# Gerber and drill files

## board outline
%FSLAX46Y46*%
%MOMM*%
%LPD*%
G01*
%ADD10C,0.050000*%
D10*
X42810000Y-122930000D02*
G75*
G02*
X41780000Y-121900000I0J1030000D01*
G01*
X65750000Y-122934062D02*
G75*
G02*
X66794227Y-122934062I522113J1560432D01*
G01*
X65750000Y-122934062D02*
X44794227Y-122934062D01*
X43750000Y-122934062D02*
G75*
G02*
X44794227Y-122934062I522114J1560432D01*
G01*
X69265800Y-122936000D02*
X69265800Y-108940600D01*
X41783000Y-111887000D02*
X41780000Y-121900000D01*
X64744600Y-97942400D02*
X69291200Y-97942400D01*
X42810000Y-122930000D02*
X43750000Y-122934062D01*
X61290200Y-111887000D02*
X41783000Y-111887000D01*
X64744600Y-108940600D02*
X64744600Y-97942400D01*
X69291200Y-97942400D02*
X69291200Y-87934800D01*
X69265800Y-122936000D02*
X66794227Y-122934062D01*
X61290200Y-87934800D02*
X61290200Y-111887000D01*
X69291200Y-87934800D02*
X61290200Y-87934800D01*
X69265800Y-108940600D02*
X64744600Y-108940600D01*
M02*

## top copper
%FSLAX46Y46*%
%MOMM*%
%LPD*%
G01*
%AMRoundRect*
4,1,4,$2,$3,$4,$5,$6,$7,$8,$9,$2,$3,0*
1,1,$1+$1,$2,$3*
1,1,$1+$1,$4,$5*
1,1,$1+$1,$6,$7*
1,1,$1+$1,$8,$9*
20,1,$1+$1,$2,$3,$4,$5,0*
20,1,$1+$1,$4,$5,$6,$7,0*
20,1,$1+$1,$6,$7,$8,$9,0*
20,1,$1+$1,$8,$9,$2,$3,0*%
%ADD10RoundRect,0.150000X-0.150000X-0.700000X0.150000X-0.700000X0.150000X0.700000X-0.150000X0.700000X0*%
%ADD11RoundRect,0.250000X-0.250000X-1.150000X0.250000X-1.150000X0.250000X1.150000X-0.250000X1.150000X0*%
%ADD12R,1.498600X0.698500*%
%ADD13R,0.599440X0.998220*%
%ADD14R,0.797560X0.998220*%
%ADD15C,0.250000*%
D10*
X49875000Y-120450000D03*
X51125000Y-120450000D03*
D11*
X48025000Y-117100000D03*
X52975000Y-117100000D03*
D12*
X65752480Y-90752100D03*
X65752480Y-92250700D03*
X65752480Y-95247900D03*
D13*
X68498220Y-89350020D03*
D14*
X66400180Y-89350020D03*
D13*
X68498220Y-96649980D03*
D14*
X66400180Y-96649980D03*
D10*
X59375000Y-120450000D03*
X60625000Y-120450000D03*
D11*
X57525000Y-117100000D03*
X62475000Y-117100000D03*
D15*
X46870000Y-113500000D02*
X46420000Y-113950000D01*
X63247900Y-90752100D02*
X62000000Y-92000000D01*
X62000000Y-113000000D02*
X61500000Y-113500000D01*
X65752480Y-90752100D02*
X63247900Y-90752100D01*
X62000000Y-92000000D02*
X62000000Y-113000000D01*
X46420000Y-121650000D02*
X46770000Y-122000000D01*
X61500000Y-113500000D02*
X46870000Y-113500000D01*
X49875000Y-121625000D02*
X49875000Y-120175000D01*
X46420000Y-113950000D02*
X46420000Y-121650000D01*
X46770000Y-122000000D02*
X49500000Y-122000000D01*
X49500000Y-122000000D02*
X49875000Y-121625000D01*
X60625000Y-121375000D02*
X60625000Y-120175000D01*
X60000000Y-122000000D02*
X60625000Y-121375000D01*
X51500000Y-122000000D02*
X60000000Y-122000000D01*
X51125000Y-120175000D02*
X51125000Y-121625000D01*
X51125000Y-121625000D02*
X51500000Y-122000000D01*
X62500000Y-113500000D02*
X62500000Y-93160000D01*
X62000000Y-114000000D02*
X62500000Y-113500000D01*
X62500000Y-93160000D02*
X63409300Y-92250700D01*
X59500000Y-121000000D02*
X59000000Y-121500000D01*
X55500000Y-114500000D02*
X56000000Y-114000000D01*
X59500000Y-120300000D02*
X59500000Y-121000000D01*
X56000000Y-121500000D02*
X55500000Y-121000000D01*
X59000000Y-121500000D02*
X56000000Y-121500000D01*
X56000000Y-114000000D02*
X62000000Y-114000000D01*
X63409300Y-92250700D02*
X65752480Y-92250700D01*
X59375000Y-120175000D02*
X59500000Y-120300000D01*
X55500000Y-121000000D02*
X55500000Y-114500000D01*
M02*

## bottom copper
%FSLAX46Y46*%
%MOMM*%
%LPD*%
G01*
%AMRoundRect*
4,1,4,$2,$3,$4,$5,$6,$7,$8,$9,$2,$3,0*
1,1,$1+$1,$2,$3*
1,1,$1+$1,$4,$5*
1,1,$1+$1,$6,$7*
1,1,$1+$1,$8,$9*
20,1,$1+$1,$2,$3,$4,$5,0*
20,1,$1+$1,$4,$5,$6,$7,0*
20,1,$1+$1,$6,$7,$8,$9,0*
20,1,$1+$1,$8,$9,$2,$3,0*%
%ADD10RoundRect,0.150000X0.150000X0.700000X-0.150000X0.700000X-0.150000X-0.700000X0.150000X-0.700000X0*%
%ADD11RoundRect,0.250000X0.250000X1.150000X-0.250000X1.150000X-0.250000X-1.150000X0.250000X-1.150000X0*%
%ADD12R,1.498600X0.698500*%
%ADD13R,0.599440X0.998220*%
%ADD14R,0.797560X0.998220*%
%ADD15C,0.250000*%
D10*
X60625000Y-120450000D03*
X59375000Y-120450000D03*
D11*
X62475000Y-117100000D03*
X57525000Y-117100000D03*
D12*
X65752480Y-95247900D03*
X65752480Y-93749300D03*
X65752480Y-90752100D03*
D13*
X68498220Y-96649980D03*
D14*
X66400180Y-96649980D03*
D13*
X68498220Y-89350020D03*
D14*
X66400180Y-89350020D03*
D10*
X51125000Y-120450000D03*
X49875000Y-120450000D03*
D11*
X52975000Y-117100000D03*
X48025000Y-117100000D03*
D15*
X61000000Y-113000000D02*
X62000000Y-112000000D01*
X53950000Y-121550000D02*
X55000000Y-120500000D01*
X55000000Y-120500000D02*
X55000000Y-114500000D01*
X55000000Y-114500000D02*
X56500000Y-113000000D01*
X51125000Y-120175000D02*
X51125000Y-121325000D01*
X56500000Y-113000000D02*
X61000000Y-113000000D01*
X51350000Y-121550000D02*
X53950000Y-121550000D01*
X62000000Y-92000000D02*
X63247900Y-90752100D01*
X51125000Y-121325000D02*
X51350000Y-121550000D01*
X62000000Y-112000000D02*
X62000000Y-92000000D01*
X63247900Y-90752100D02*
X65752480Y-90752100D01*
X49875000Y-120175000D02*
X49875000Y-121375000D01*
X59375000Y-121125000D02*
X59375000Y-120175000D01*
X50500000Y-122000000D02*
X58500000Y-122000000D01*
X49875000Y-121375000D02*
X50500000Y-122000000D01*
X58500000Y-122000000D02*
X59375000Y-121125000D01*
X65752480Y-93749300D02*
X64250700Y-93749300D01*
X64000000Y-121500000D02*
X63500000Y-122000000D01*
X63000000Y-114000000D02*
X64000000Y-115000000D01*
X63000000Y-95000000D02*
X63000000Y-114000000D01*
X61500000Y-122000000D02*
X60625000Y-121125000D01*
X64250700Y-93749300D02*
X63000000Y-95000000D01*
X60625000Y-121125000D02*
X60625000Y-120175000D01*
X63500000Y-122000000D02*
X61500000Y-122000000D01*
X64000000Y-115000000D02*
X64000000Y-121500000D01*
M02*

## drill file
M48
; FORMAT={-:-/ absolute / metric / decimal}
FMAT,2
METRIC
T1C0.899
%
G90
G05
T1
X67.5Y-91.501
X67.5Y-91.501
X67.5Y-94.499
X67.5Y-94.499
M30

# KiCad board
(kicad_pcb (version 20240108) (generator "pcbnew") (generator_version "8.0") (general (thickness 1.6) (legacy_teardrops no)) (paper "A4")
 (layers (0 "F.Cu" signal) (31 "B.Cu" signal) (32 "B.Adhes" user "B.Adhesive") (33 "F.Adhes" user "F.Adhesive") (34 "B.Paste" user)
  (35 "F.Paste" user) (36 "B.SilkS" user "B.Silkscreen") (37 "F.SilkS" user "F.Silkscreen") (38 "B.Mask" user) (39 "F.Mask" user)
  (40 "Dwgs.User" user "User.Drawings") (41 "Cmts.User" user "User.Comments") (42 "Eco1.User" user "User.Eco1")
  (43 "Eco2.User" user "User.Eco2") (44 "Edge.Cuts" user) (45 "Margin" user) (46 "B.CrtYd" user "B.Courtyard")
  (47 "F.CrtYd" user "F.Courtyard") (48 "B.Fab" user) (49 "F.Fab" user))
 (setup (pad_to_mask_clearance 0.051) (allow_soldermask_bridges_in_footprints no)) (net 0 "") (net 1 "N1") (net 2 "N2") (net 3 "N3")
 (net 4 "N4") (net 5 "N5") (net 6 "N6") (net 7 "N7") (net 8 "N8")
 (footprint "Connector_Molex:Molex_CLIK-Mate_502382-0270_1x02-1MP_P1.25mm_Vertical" (layer "F.Cu") (at 50.5 118.5)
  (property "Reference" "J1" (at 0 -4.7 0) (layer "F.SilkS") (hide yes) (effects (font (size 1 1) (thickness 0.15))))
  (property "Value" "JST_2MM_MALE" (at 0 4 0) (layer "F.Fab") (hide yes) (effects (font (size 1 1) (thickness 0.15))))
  (pad "1" smd roundrect (at -0.625 1.95) (size 0.6 1.7) (layers "F.Cu" "F.Paste" "F.Mask") (roundrect_rratio 0.25) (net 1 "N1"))
  (pad "2" smd roundrect (at 0.625 1.95) (size 0.6 1.7) (layers "F.Cu" "F.Paste" "F.Mask") (roundrect_rratio 0.25) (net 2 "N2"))
  (pad "MP" smd roundrect (at -2.475 -1.4) (size 1 2.8) (layers "F.Cu" "F.Paste" "F.Mask") (roundrect_rratio 0.25))
  (pad "MP" smd roundrect (at 2.475 -1.4) (size 1 2.8) (layers "F.Cu" "F.Paste" "F.Mask") (roundrect_rratio 0.25)))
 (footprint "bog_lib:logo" (layer "F.Cu") (at 66.711323 112.325837)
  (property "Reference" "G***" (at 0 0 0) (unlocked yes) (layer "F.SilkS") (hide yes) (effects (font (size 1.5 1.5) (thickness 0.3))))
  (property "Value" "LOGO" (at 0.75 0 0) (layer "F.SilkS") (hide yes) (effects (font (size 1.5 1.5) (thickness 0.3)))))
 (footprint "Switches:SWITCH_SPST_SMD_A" (layer "F.Cu") (at 67.5 93 -90)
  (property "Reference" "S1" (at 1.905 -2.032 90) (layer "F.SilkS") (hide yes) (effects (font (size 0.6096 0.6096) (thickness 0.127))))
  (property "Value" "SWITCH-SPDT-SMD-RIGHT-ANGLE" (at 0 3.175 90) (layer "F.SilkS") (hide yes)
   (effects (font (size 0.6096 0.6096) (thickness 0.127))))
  (pad "" np_thru_hole circle (at -1.4986 0 270) (size 0.89916 0.89916) (drill 0.89916) (layers "*.Cu" "*.Mask") (solder_mask_margin 0.1016))
  (pad "" np_thru_hole circle (at 1.4986 0 270) (size 0.89916 0.89916) (drill 0.89916) (layers "*.Cu" "*.Mask") (solder_mask_margin 0.1016))
  (pad "1" smd rect (at -2.2479 1.74752 90) (size 0.6985 1.4986) (layers "F.Cu" "F.Paste" "F.Mask") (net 1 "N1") (solder_mask_margin 0.1016))
  (pad "2" smd rect (at -0.7493 1.74752 90) (size 0.6985 1.4986) (layers "F.Cu" "F.Paste" "F.Mask") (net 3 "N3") (solder_mask_margin 0.1016))
  (pad "3" smd rect (at 2.2479 1.74752 90) (size 0.6985 1.4986) (layers "F.Cu" "F.Paste" "F.Mask") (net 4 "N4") (solder_mask_margin 0.1016))
  (pad "GND1" smd rect (at -3.64998 -0.99822 270) (size 0.99822 0.59944) (layers "F.Cu" "F.Paste" "F.Mask") (solder_mask_margin 0.1016))
  (pad "GND2" smd rect (at -3.64998 1.09982 270) (size 0.99822 0.79756) (layers "F.Cu" "F.Paste" "F.Mask") (solder_mask_margin 0.1016))
  (pad "GND3" smd rect (at 3.64998 -0.99822 270) (size 0.99822 0.59944) (layers "F.Cu" "F.Paste" "F.Mask") (solder_mask_margin 0.1016))
  (pad "GND4" smd rect (at 3.64998 1.09982 270) (size 0.99822 0.79756) (layers "F.Cu" "F.Paste" "F.Mask") (solder_mask_margin 0.1016)))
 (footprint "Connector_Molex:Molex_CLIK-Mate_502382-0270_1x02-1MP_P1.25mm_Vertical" (layer "F.Cu") (at 60 118.5)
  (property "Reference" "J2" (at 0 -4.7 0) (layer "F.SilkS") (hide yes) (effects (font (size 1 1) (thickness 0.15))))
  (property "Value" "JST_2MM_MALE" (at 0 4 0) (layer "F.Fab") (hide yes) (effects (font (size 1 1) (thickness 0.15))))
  (pad "1" smd roundrect (at -0.625 1.95) (size 0.6 1.7) (layers "F.Cu" "F.Paste" "F.Mask") (roundrect_rratio 0.25) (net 3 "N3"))
  (pad "2" smd roundrect (at 0.625 1.95) (size 0.6 1.7) (layers "F.Cu" "F.Paste" "F.Mask") (roundrect_rratio 0.25) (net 2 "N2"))
  (pad "MP" smd roundrect (at -2.475 -1.4) (size 1 2.8) (layers "F.Cu" "F.Paste" "F.Mask") (roundrect_rratio 0.25))
  (pad "MP" smd roundrect (at 2.475 -1.4) (size 1 2.8) (layers "F.Cu" "F.Paste" "F.Mask") (roundrect_rratio 0.25)))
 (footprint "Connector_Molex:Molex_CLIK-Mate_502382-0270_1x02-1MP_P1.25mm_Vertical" (layer "B.Cu") (at 60 118.5 180)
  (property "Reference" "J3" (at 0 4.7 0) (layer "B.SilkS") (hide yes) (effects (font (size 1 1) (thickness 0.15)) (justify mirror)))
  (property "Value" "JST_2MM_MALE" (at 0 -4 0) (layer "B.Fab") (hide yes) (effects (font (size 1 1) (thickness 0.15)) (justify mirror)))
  (pad "1" smd roundrect (at -0.625 -1.95 180) (size 0.6 1.7) (layers "B.Cu" "B.Paste" "B.Mask") (roundrect_rratio 0.25) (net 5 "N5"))
  (pad "2" smd roundrect (at 0.625 -1.95 180) (size 0.6 1.7) (layers "B.Cu" "B.Paste" "B.Mask") (roundrect_rratio 0.25) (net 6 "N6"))
  (pad "MP" smd roundrect (at -2.475 1.4 180) (size 1 2.8) (layers "B.Cu" "B.Paste" "B.Mask") (roundrect_rratio 0.25))
  (pad "MP" smd roundrect (at 2.475 1.4 180) (size 1 2.8) (layers "B.Cu" "B.Paste" "B.Mask") (roundrect_rratio 0.25)))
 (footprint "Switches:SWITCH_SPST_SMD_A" (layer "B.Cu") (at 67.5 93 90)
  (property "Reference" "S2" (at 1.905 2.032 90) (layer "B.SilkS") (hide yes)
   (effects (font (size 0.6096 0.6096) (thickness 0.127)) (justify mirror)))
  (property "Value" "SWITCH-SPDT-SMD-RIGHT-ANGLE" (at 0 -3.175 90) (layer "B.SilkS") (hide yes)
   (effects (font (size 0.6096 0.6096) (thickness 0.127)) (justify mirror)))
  (pad "" np_thru_hole circle (at -1.4986 0 90) (size 0.89916 0.89916) (drill 0.89916) (layers "*.Cu" "*.Mask") (solder_mask_margin 0.1016))
  (pad "" np_thru_hole circle (at 1.4986 0 90) (size 0.89916 0.89916) (drill 0.89916) (layers "*.Cu" "*.Mask") (solder_mask_margin 0.1016))
  (pad "1" smd rect (at -2.2479 -1.74752 270) (size 0.6985 1.4986) (layers "B.Cu" "B.Paste" "B.Mask") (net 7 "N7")
   (solder_mask_margin 0.1016))
  (pad "2" smd rect (at -0.7493 -1.74752 270) (size 0.6985 1.4986) (layers "B.Cu" "B.Paste" "B.Mask") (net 5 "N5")
   (solder_mask_margin 0.1016))
  (pad "3" smd rect (at 2.2479 -1.74752 270) (size 0.6985 1.4986) (layers "B.Cu" "B.Paste" "B.Mask") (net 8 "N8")
   (solder_mask_margin 0.1016))
  (pad "GND1" smd rect (at -3.64998 0.99822 90) (size 0.99822 0.59944) (layers "B.Cu" "B.Paste" "B.Mask") (solder_mask_margin 0.1016))
  (pad "GND2" smd rect (at -3.64998 -1.09982 90) (size 0.99822 0.79756) (layers "B.Cu" "B.Paste" "B.Mask") (solder_mask_margin 0.1016))
  (pad "GND3" smd rect (at 3.64998 0.99822 90) (size 0.99822 0.59944) (layers "B.Cu" "B.Paste" "B.Mask") (solder_mask_margin 0.1016))
  (pad "GND4" smd rect (at 3.64998 -1.09982 90) (size 0.99822 0.79756) (layers "B.Cu" "B.Paste" "B.Mask") (solder_mask_margin 0.1016)))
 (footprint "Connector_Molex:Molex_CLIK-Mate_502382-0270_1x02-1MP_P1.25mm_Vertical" (layer "B.Cu") (at 50.5 118.5 180)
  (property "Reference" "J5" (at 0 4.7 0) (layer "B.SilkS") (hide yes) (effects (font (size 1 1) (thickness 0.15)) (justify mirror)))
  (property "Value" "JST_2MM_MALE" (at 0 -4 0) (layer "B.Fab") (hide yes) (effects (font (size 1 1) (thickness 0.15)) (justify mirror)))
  (pad "1" smd roundrect (at -0.625 -1.95 180) (size 0.6 1.7) (layers "B.Cu" "B.Paste" "B.Mask") (roundrect_rratio 0.25) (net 8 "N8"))
  (pad "2" smd roundrect (at 0.625 -1.95 180) (size 0.6 1.7) (layers "B.Cu" "B.Paste" "B.Mask") (roundrect_rratio 0.25) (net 6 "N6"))
  (pad "MP" smd roundrect (at -2.475 1.4 180) (size 1 2.8) (layers "B.Cu" "B.Paste" "B.Mask") (roundrect_rratio 0.25))
  (pad "MP" smd roundrect (at 2.475 1.4 180) (size 1 2.8) (layers "B.Cu" "B.Paste" "B.Mask") (roundrect_rratio 0.25)))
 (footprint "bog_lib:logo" (layer "B.Cu") (at 67.051126 112.325837 180)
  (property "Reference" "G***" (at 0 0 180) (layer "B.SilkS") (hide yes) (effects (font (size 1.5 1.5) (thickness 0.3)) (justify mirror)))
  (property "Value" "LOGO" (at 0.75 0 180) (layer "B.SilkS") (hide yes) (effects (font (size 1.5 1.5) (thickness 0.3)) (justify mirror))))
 (gr_arc (start 42.81 122.93) (mid 42.08168 122.62832) (end 41.78 121.9) (stroke (width 0.05) (type default)) (layer "Edge.Cuts"))
 (gr_arc (start 65.75 122.934062) (mid 66.272114 119.728166) (end 66.794227 122.934062) (stroke (width 0.05) (type solid))
  (layer "Edge.Cuts"))
 (gr_line (start 65.75 122.934062) (end 44.794227 122.934062) (stroke (width 0.05) (type solid)) (layer "Edge.Cuts"))
 (gr_arc (start 43.75 122.934062) (mid 44.272114 119.728166) (end 44.794227 122.934062) (stroke (width 0.05) (type solid))
  (layer "Edge.Cuts"))
 (gr_line (start 69.2658 122.936) (end 69.2658 108.9406) (stroke (width 0.05) (type solid)) (layer "Edge.Cuts"))
 (gr_line (start 41.783 111.887) (end 41.78 121.9) (stroke (width 0.05) (type solid)) (layer "Edge.Cuts"))
 (gr_line (start 64.7446 97.9424) (end 69.2912 97.9424) (stroke (width 0.05) (type solid)) (layer "Edge.Cuts"))
 (gr_line (start 42.81 122.93) (end 43.75 122.934062) (stroke (width 0.05) (type solid)) (layer "Edge.Cuts"))
 (gr_line (start 61.2902 111.887) (end 41.783 111.887) (stroke (width 0.05) (type solid)) (layer "Edge.Cuts"))
 (gr_line (start 64.7446 108.9406) (end 64.7446 97.9424) (stroke (width 0.05) (type solid)) (layer "Edge.Cuts"))
 (gr_line (start 69.2912 97.9424) (end 69.2912 87.9348) (stroke (width 0.05) (type solid)) (layer "Edge.Cuts"))
 (gr_line (start 69.2658 122.936) (end 66.794227 122.934062) (stroke (width 0.05) (type solid)) (layer "Edge.Cuts"))
 (gr_line (start 61.2902 87.9348) (end 61.2902 111.887) (stroke (width 0.05) (type solid)) (layer "Edge.Cuts"))
 (gr_line (start 69.2912 87.9348) (end 61.2902 87.9348) (stroke (width 0.05) (type solid)) (layer "Edge.Cuts"))
 (gr_line (start 69.2658 108.9406) (end 64.7446 108.9406) (stroke (width 0.05) (type solid)) (layer "Edge.Cuts"))
 (segment (start 46.87 113.5) (end 46.42 113.95) (width 0.25) (layer "F.Cu") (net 1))
 (segment (start 63.2479 90.7521) (end 62 92) (width 0.25) (layer "F.Cu") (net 1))
 (segment (start 62 113) (end 61.5 113.5) (width 0.25) (layer "F.Cu") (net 1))
 (segment (start 65.75248 90.7521) (end 63.2479 90.7521) (width 0.25) (layer "F.Cu") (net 1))
 (segment (start 62 92) (end 62 113) (width 0.25) (layer "F.Cu") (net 1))
 (segment (start 46.42 121.65) (end 46.77 122) (width 0.25) (layer "F.Cu") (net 1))
 (segment (start 61.5 113.5) (end 46.87 113.5) (width 0.25) (layer "F.Cu") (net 1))
 (segment (start 49.875 121.625) (end 49.875 120.175) (width 0.25) (layer "F.Cu") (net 1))
 (segment (start 46.42 113.95) (end 46.42 121.65) (width 0.25) (layer "F.Cu") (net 1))
 (segment (start 46.77 122) (end 49.5 122) (width 0.25) (layer "F.Cu") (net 1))
 (segment (start 49.5 122) (end 49.875 121.625) (width 0.25) (layer "F.Cu") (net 1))
 (segment (start 60.625 121.375) (end 60.625 120.175) (width 0.25) (layer "F.Cu") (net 2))
 (segment (start 60 122) (end 60.625 121.375) (width 0.25) (layer "F.Cu") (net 2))
 (segment (start 51.5 122) (end 60 122) (width 0.25) (layer "F.Cu") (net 2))
 (segment (start 51.125 120.175) (end 51.125 121.625) (width 0.25) (layer "F.Cu") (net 2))
 (segment (start 51.125 121.625) (end 51.5 122) (width 0.25) (layer "F.Cu") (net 2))
 (segment (start 62.5 113.5) (end 62.5 93.16) (width 0.25) (layer "F.Cu") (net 3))
 (segment (start 62 114) (end 62.5 113.5) (width 0.25) (layer "F.Cu") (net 3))
 (segment (start 62.5 93.16) (end 63.4093 92.2507) (width 0.25) (layer "F.Cu") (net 3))
 (segment (start 59.5 121) (end 59 121.5) (width 0.25) (layer "F.Cu") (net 3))
 (segment (start 55.5 114.5) (end 56 114) (width 0.25) (layer "F.Cu") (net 3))
 (segment (start 59.5 120.3) (end 59.5 121) (width 0.25) (layer "F.Cu") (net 3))
 (segment (start 56 121.5) (end 55.5 121) (width 0.25) (layer "F.Cu") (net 3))
 (segment (start 59 121.5) (end 56 121.5) (width 0.25) (layer "F.Cu") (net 3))
 (segment (start 56 114) (end 62 114) (width 0.25) (layer "F.Cu") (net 3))
 (segment (start 63.4093 92.2507) (end 65.75248 92.2507) (width 0.25) (layer "F.Cu") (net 3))
 (segment (start 59.375 120.175) (end 59.5 120.3) (width 0.25) (layer "F.Cu") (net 3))
 (segment (start 55.5 121) (end 55.5 114.5) (width 0.25) (layer "F.Cu") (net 3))
 (segment (start 61 113) (end 62 112) (width 0.25) (layer "B.Cu") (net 8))
 (segment (start 53.95 121.55) (end 55 120.5) (width 0.25) (layer "B.Cu") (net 8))
 (segment (start 55 120.5) (end 55 114.5) (width 0.25) (layer "B.Cu") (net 8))
 (segment (start 55 114.5) (end 56.5 113) (width 0.25) (layer "B.Cu") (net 8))
 (segment (start 51.125 120.175) (end 51.125 121.325) (width 0.25) (layer "B.Cu") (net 8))
 (segment (start 56.5 113) (end 61 113) (width 0.25) (layer "B.Cu") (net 8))
 (segment (start 51.35 121.55) (end 53.95 121.55) (width 0.25) (layer "B.Cu") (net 8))
 (segment (start 62 92) (end 63.2479 90.7521) (width 0.25) (layer "B.Cu") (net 8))
 (segment (start 51.125 121.325) (end 51.35 121.55) (width 0.25) (layer "B.Cu") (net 8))
 (segment (start 62 112) (end 62 92) (width 0.25) (layer "B.Cu") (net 8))
 (segment (start 63.2479 90.7521) (end 65.75248 90.7521) (width 0.25) (layer "B.Cu") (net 8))
 (segment (start 49.875 120.175) (end 49.875 121.375) (width 0.25) (layer "B.Cu") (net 6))
 (segment (start 59.375 121.125) (end 59.375 120.175) (width 0.25) (layer "B.Cu") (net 6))
 (segment (start 50.5 122) (end 58.5 122) (width 0.25) (layer "B.Cu") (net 6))
 (segment (start 49.875 121.375) (end 50.5 122) (width 0.25) (layer "B.Cu") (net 6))
 (segment (start 58.5 122) (end 59.375 121.125) (width 0.25) (layer "B.Cu") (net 6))
 (segment (start 65.75248 93.7493) (end 64.2507 93.7493) (width 0.25) (layer "B.Cu") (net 5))
 (segment (start 64 121.5) (end 63.5 122) (width 0.25) (layer "B.Cu") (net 5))
 (segment (start 63 114) (end 64 115) (width 0.25) (layer "B.Cu") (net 5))
 (segment (start 63 95) (end 63 114) (width 0.25) (layer "B.Cu") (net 5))
 (segment (start 61.5 122) (end 60.625 121.125) (width 0.25) (layer "B.Cu") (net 5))
 (segment (start 64.2507 93.7493) (end 63 95) (width 0.25) (layer "B.Cu") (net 5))
 (segment (start 60.625 121.125) (end 60.625 120.175) (width 0.25) (layer "B.Cu") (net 5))
 (segment (start 63.5 122) (end 61.5 122) (width 0.25) (layer "B.Cu") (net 5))
 (segment (start 64 115) (end 64 121.5) (width 0.25) (layer "B.Cu") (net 5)))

